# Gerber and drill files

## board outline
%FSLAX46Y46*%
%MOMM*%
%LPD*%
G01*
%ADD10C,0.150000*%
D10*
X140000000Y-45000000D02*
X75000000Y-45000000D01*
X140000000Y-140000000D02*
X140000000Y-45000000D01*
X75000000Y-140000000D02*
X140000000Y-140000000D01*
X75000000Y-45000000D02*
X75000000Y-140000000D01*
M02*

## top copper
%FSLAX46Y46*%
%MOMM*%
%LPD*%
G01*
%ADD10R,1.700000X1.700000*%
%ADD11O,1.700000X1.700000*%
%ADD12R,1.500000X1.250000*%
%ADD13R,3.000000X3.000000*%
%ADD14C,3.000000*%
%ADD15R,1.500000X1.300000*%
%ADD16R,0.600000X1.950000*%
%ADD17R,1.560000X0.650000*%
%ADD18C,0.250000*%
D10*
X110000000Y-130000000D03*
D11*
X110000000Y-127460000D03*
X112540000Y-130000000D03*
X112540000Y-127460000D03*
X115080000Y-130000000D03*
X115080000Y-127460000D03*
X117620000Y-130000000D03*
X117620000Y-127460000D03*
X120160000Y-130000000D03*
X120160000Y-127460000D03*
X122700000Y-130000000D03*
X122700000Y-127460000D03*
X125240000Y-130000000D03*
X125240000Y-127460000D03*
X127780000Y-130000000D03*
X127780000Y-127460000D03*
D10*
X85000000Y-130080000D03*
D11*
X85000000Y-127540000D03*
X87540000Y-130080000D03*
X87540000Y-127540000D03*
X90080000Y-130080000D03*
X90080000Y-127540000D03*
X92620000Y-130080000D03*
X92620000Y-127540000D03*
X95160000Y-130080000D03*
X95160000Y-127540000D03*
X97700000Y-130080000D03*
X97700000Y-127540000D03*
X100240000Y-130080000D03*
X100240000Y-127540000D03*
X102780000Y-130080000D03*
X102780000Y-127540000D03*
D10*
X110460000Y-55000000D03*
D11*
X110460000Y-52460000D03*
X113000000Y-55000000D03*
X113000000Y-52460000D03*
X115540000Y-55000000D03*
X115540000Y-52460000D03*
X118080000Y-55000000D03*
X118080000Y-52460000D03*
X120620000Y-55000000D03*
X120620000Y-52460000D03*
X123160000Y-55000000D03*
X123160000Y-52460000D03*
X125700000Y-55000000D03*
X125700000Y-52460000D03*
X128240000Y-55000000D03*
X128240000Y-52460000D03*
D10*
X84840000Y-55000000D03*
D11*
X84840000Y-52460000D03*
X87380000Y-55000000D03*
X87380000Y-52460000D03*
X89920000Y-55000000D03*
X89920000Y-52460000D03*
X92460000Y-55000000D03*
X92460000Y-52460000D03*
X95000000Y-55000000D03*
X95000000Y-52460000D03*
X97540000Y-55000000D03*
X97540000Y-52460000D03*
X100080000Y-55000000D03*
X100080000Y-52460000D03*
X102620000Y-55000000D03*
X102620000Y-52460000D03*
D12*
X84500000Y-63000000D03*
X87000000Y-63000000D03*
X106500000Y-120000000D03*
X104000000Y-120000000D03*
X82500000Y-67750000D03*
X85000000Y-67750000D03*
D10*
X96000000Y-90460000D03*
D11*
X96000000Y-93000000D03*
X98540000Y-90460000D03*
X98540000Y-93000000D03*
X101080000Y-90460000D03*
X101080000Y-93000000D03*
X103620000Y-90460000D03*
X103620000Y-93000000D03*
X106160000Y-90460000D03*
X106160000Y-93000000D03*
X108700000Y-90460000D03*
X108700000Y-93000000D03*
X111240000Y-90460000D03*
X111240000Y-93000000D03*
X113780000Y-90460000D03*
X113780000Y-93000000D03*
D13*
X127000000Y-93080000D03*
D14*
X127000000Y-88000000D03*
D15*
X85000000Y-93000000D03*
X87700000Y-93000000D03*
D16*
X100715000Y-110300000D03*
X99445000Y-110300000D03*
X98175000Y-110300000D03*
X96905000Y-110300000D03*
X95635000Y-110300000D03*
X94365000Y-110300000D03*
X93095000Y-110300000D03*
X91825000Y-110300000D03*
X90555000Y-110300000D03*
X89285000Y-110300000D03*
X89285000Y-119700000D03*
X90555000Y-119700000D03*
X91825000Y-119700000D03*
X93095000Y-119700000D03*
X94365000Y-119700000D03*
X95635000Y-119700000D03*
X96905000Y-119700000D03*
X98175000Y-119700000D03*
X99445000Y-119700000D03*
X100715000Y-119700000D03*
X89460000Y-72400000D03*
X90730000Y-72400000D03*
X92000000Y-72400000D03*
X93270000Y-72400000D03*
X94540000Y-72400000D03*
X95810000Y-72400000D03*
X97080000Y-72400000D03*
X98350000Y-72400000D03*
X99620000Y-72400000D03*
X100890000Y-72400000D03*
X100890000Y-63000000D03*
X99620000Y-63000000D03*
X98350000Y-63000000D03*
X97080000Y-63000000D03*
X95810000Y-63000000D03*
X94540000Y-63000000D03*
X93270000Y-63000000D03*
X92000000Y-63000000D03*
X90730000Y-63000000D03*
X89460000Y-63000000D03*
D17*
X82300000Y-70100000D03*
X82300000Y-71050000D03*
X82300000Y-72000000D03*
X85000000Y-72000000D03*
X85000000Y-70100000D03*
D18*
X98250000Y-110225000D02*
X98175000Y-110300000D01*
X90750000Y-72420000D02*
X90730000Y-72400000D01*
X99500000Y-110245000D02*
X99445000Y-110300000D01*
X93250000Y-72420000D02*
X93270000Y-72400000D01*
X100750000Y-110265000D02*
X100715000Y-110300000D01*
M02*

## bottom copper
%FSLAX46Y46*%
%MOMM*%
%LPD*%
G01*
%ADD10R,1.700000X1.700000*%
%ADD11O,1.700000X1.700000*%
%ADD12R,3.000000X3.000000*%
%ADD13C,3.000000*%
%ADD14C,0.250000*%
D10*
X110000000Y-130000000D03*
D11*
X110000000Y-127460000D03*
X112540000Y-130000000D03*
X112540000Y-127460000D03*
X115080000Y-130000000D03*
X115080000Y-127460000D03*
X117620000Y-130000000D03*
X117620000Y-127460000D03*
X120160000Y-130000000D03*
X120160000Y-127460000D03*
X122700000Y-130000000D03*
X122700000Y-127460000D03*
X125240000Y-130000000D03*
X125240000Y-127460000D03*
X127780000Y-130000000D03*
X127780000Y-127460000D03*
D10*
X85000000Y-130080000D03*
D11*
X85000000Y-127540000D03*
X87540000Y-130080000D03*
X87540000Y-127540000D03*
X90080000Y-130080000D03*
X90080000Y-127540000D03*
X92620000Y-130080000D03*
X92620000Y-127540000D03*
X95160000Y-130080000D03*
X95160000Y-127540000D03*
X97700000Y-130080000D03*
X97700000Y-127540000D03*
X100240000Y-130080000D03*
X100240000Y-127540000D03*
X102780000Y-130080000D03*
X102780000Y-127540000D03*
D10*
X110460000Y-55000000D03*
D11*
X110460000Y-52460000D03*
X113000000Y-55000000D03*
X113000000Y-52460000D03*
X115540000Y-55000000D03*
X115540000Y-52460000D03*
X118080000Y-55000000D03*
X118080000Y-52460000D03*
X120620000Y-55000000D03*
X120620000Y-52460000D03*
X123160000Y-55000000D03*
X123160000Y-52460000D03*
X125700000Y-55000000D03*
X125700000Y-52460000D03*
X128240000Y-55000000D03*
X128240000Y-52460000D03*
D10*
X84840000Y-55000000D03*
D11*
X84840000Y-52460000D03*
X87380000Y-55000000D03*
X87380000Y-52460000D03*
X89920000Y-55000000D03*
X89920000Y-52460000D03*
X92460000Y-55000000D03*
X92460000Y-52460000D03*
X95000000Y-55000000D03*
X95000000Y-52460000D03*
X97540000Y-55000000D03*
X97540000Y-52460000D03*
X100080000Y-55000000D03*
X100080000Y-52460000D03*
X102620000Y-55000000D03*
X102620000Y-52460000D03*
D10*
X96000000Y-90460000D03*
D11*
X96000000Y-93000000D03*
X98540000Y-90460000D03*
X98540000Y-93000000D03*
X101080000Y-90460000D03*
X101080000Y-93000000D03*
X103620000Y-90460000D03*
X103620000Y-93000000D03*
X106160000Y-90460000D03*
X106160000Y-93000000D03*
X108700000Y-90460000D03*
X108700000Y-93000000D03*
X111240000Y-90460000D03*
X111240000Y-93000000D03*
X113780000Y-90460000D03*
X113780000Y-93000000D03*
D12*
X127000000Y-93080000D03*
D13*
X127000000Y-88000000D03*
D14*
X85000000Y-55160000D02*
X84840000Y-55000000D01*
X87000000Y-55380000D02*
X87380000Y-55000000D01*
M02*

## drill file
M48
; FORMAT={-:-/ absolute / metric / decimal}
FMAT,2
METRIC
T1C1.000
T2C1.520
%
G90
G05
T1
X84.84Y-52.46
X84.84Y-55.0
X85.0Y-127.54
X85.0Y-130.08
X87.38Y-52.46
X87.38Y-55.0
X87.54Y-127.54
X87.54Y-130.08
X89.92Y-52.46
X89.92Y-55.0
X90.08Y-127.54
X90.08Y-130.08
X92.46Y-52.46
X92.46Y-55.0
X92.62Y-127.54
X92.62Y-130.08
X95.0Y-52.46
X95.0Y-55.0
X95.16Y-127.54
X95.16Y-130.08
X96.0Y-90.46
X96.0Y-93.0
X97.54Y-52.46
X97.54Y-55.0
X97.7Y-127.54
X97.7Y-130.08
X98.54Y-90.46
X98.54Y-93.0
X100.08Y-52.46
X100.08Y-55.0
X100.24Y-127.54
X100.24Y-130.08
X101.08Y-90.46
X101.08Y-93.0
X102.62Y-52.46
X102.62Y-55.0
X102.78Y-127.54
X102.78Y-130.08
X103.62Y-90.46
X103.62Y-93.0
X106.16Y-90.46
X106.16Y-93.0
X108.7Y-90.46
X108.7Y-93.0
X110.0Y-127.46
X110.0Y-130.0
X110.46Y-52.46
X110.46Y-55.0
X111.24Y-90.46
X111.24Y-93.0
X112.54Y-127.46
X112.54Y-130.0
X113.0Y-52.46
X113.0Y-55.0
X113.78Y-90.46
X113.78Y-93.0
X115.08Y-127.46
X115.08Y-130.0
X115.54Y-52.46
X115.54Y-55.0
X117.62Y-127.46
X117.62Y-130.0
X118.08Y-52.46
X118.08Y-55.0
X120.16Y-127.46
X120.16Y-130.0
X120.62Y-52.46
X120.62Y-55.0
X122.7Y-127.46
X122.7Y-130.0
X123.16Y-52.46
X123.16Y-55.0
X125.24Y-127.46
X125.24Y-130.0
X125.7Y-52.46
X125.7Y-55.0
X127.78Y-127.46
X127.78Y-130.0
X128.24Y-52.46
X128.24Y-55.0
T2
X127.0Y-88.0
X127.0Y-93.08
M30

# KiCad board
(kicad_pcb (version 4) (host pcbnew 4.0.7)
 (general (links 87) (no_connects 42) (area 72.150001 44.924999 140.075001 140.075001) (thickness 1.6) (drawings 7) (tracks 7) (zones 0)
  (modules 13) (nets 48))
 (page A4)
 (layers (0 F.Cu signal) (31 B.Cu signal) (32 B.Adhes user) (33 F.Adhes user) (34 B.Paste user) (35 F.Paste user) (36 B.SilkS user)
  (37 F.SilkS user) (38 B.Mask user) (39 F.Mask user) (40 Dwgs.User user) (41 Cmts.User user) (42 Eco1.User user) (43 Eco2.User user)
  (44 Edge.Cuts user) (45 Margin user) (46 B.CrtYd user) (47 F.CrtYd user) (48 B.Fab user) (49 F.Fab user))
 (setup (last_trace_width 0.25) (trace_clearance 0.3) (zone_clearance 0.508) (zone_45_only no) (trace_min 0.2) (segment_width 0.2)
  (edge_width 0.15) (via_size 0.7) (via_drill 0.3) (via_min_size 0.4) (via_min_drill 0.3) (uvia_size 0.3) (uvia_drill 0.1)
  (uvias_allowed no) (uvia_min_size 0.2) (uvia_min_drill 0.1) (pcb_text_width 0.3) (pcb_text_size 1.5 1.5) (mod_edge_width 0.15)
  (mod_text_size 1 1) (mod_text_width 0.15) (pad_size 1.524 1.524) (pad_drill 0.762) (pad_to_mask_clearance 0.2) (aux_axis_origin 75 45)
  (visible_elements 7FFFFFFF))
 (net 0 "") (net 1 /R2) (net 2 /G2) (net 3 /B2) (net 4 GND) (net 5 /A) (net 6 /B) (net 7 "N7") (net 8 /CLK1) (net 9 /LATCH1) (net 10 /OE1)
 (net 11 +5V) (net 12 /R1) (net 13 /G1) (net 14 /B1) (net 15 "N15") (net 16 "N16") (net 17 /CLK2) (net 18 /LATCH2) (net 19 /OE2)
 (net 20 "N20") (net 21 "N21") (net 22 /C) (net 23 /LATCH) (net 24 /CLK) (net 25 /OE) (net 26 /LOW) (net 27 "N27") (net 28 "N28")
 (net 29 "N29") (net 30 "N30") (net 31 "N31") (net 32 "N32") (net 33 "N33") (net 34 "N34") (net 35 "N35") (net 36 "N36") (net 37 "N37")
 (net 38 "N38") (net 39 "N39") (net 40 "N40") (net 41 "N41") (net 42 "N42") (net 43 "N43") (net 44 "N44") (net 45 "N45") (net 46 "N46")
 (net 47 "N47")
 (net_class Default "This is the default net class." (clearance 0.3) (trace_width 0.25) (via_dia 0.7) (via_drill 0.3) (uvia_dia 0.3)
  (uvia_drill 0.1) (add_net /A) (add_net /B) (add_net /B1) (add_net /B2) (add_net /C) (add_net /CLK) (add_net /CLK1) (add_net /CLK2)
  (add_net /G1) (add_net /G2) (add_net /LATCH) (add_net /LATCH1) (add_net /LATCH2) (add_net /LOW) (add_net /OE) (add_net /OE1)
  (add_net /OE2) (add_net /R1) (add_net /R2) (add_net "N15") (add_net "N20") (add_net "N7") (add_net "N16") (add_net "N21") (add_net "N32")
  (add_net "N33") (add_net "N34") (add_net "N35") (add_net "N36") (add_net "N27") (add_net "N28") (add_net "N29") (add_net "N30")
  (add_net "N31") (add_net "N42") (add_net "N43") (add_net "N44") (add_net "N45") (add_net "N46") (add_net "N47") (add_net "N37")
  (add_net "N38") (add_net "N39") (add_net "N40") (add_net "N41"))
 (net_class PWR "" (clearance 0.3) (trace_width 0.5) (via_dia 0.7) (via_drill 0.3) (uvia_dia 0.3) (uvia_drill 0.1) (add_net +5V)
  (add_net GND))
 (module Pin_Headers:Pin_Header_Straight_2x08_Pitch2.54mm (layer F.Cu) (at 110 130 90)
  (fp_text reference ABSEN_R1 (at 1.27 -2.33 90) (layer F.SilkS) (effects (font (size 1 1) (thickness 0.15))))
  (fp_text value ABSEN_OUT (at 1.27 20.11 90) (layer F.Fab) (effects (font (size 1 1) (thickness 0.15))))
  (pad 1 thru_hole rect (at 0 0 90) (size 1.7 1.7) (drill 1) (layers *.Cu *.Mask) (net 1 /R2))
  (pad 2 thru_hole oval (at 2.54 0 90) (size 1.7 1.7) (drill 1) (layers *.Cu *.Mask) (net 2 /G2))
  (pad 3 thru_hole oval (at 0 2.54 90) (size 1.7 1.7) (drill 1) (layers *.Cu *.Mask) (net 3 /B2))
  (pad 4 thru_hole oval (at 2.54 2.54 90) (size 1.7 1.7) (drill 1) (layers *.Cu *.Mask) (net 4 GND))
  (pad 5 thru_hole oval (at 0 5.08 90) (size 1.7 1.7) (drill 1) (layers *.Cu *.Mask) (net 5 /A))
  (pad 6 thru_hole oval (at 2.54 5.08 90) (size 1.7 1.7) (drill 1) (layers *.Cu *.Mask) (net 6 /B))
  (pad 7 thru_hole oval (at 0 7.62 90) (size 1.7 1.7) (drill 1) (layers *.Cu *.Mask) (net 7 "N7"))
  (pad 8 thru_hole oval (at 2.54 7.62 90) (size 1.7 1.7) (drill 1) (layers *.Cu *.Mask) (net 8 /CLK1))
  (pad 9 thru_hole oval (at 0 10.16 90) (size 1.7 1.7) (drill 1) (layers *.Cu *.Mask) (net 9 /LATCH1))
  (pad 10 thru_hole oval (at 2.54 10.16 90) (size 1.7 1.7) (drill 1) (layers *.Cu *.Mask) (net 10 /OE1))
  (pad 11 thru_hole oval (at 0 12.7 90) (size 1.7 1.7) (drill 1) (layers *.Cu *.Mask) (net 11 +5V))
  (pad 12 thru_hole oval (at 2.54 12.7 90) (size 1.7 1.7) (drill 1) (layers *.Cu *.Mask) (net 4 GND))
  (pad 13 thru_hole oval (at 0 15.24 90) (size 1.7 1.7) (drill 1) (layers *.Cu *.Mask) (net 11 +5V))
  (pad 14 thru_hole oval (at 2.54 15.24 90) (size 1.7 1.7) (drill 1) (layers *.Cu *.Mask) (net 4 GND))
  (pad 15 thru_hole oval (at 0 17.78 90) (size 1.7 1.7) (drill 1) (layers *.Cu *.Mask) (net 11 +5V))
  (pad 16 thru_hole oval (at 2.54 17.78 90) (size 1.7 1.7) (drill 1) (layers *.Cu *.Mask) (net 4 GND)))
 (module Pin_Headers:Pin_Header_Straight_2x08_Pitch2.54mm (layer F.Cu) (at 85 130.08 90)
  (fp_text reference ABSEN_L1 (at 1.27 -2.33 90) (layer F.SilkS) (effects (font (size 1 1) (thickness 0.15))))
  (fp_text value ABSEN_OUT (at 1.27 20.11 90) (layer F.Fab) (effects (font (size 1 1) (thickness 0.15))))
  (pad 1 thru_hole rect (at 0 0 90) (size 1.7 1.7) (drill 1) (layers *.Cu *.Mask) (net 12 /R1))
  (pad 2 thru_hole oval (at 2.54 0 90) (size 1.7 1.7) (drill 1) (layers *.Cu *.Mask) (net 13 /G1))
  (pad 3 thru_hole oval (at 0 2.54 90) (size 1.7 1.7) (drill 1) (layers *.Cu *.Mask) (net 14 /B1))
  (pad 4 thru_hole oval (at 2.54 2.54 90) (size 1.7 1.7) (drill 1) (layers *.Cu *.Mask) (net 4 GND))
  (pad 5 thru_hole oval (at 0 5.08 90) (size 1.7 1.7) (drill 1) (layers *.Cu *.Mask) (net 5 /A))
  (pad 6 thru_hole oval (at 2.54 5.08 90) (size 1.7 1.7) (drill 1) (layers *.Cu *.Mask) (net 6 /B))
  (pad 7 thru_hole oval (at 0 7.62 90) (size 1.7 1.7) (drill 1) (layers *.Cu *.Mask) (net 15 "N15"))
  (pad 8 thru_hole oval (at 2.54 7.62 90) (size 1.7 1.7) (drill 1) (layers *.Cu *.Mask) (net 8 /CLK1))
  (pad 9 thru_hole oval (at 0 10.16 90) (size 1.7 1.7) (drill 1) (layers *.Cu *.Mask) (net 9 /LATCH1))
  (pad 10 thru_hole oval (at 2.54 10.16 90) (size 1.7 1.7) (drill 1) (layers *.Cu *.Mask) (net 10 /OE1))
  (pad 11 thru_hole oval (at 0 12.7 90) (size 1.7 1.7) (drill 1) (layers *.Cu *.Mask) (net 11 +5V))
  (pad 12 thru_hole oval (at 2.54 12.7 90) (size 1.7 1.7) (drill 1) (layers *.Cu *.Mask) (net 4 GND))
  (pad 13 thru_hole oval (at 0 15.24 90) (size 1.7 1.7) (drill 1) (layers *.Cu *.Mask) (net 11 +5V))
  (pad 14 thru_hole oval (at 2.54 15.24 90) (size 1.7 1.7) (drill 1) (layers *.Cu *.Mask) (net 4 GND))
  (pad 15 thru_hole oval (at 0 17.78 90) (size 1.7 1.7) (drill 1) (layers *.Cu *.Mask) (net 11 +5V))
  (pad 16 thru_hole oval (at 2.54 17.78 90) (size 1.7 1.7) (drill 1) (layers *.Cu *.Mask) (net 4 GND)))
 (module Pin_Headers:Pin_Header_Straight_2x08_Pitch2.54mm (layer F.Cu) (at 110.46 55 90)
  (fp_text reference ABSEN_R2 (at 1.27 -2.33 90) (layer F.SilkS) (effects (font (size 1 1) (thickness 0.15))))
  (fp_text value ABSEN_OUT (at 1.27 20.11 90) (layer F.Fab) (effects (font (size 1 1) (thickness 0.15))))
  (pad 1 thru_hole rect (at 0 0 90) (size 1.7 1.7) (drill 1) (layers *.Cu *.Mask) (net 1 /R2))
  (pad 2 thru_hole oval (at 2.54 0 90) (size 1.7 1.7) (drill 1) (layers *.Cu *.Mask) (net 2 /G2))
  (pad 3 thru_hole oval (at 0 2.54 90) (size 1.7 1.7) (drill 1) (layers *.Cu *.Mask) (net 3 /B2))
  (pad 4 thru_hole oval (at 2.54 2.54 90) (size 1.7 1.7) (drill 1) (layers *.Cu *.Mask) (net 4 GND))
  (pad 5 thru_hole oval (at 0 5.08 90) (size 1.7 1.7) (drill 1) (layers *.Cu *.Mask) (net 5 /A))
  (pad 6 thru_hole oval (at 2.54 5.08 90) (size 1.7 1.7) (drill 1) (layers *.Cu *.Mask) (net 6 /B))
  (pad 7 thru_hole oval (at 0 7.62 90) (size 1.7 1.7) (drill 1) (layers *.Cu *.Mask) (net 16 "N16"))
  (pad 8 thru_hole oval (at 2.54 7.62 90) (size 1.7 1.7) (drill 1) (layers *.Cu *.Mask) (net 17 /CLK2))
  (pad 9 thru_hole oval (at 0 10.16 90) (size 1.7 1.7) (drill 1) (layers *.Cu *.Mask) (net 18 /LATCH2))
  (pad 10 thru_hole oval (at 2.54 10.16 90) (size 1.7 1.7) (drill 1) (layers *.Cu *.Mask) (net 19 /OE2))
  (pad 11 thru_hole oval (at 0 12.7 90) (size 1.7 1.7) (drill 1) (layers *.Cu *.Mask) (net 11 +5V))
  (pad 12 thru_hole oval (at 2.54 12.7 90) (size 1.7 1.7) (drill 1) (layers *.Cu *.Mask) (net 4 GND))
  (pad 13 thru_hole oval (at 0 15.24 90) (size 1.7 1.7) (drill 1) (layers *.Cu *.Mask) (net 11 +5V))
  (pad 14 thru_hole oval (at 2.54 15.24 90) (size 1.7 1.7) (drill 1) (layers *.Cu *.Mask) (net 4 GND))
  (pad 15 thru_hole oval (at 0 17.78 90) (size 1.7 1.7) (drill 1) (layers *.Cu *.Mask) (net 11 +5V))
  (pad 16 thru_hole oval (at 2.54 17.78 90) (size 1.7 1.7) (drill 1) (layers *.Cu *.Mask) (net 4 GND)))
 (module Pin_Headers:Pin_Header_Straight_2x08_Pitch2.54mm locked (layer F.Cu) (at 84.84 55 90)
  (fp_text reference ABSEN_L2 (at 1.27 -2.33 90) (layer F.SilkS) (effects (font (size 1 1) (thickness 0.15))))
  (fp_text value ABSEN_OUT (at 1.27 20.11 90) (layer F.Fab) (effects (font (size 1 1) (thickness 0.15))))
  (pad 1 thru_hole rect (at 0 0 90) (size 1.7 1.7) (drill 1) (layers *.Cu *.Mask) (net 12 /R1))
  (pad 2 thru_hole oval (at 2.54 0 90) (size 1.7 1.7) (drill 1) (layers *.Cu *.Mask) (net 13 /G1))
  (pad 3 thru_hole oval (at 0 2.54 90) (size 1.7 1.7) (drill 1) (layers *.Cu *.Mask) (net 14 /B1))
  (pad 4 thru_hole oval (at 2.54 2.54 90) (size 1.7 1.7) (drill 1) (layers *.Cu *.Mask) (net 4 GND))
  (pad 5 thru_hole oval (at 0 5.08 90) (size 1.7 1.7) (drill 1) (layers *.Cu *.Mask) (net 5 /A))
  (pad 6 thru_hole oval (at 2.54 5.08 90) (size 1.7 1.7) (drill 1) (layers *.Cu *.Mask) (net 6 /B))
  (pad 7 thru_hole oval (at 0 7.62 90) (size 1.7 1.7) (drill 1) (layers *.Cu *.Mask) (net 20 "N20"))
  (pad 8 thru_hole oval (at 2.54 7.62 90) (size 1.7 1.7) (drill 1) (layers *.Cu *.Mask) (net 17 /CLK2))
  (pad 9 thru_hole oval (at 0 10.16 90) (size 1.7 1.7) (drill 1) (layers *.Cu *.Mask) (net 18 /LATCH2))
  (pad 10 thru_hole oval (at 2.54 10.16 90) (size 1.7 1.7) (drill 1) (layers *.Cu *.Mask) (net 19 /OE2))
  (pad 11 thru_hole oval (at 0 12.7 90) (size 1.7 1.7) (drill 1) (layers *.Cu *.Mask) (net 11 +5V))
  (pad 12 thru_hole oval (at 2.54 12.7 90) (size 1.7 1.7) (drill 1) (layers *.Cu *.Mask) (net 4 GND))
  (pad 13 thru_hole oval (at 0 15.24 90) (size 1.7 1.7) (drill 1) (layers *.Cu *.Mask) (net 11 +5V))
  (pad 14 thru_hole oval (at 2.54 15.24 90) (size 1.7 1.7) (drill 1) (layers *.Cu *.Mask) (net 4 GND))
  (pad 15 thru_hole oval (at 0 17.78 90) (size 1.7 1.7) (drill 1) (layers *.Cu *.Mask) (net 11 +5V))
  (pad 16 thru_hole oval (at 2.54 17.78 90) (size 1.7 1.7) (drill 1) (layers *.Cu *.Mask) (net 4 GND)))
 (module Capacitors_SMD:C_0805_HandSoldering (layer F.Cu) (at 85.75 63)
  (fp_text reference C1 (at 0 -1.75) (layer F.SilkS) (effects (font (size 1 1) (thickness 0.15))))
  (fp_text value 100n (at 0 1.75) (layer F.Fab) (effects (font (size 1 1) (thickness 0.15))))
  (pad 1 smd rect (at -1.25 0) (size 1.5 1.25) (layers F.Cu F.Paste F.Mask) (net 4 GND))
  (pad 2 smd rect (at 1.25 0) (size 1.5 1.25) (layers F.Cu F.Paste F.Mask) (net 11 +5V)))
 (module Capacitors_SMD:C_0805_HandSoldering (layer F.Cu) (at 105.25 120 180)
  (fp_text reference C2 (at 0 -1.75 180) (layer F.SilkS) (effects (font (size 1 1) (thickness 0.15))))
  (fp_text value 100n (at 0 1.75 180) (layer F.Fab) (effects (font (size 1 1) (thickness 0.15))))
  (pad 1 smd rect (at -1.25 0 180) (size 1.5 1.25) (layers F.Cu F.Paste F.Mask) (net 4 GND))
  (pad 2 smd rect (at 1.25 0 180) (size 1.5 1.25) (layers F.Cu F.Paste F.Mask) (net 11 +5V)))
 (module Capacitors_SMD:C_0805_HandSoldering (layer F.Cu) (at 83.75 67.75)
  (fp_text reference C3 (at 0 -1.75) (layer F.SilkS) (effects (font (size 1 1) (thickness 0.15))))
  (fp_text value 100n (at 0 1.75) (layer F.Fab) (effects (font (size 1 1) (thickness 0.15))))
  (pad 1 smd rect (at -1.25 0) (size 1.5 1.25) (layers F.Cu F.Paste F.Mask) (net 4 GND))
  (pad 2 smd rect (at 1.25 0) (size 1.5 1.25) (layers F.Cu F.Paste F.Mask) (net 11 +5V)))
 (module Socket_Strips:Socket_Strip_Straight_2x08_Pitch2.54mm (layer F.Cu) (at 96 90.46 90)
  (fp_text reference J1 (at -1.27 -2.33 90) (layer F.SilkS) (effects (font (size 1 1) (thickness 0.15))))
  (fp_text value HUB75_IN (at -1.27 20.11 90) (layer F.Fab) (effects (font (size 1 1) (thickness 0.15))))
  (pad 1 thru_hole rect (at 0 0 90) (size 1.7 1.7) (drill 1) (layers *.Cu *.Mask) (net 13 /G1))
  (pad 2 thru_hole oval (at -2.54 0 90) (size 1.7 1.7) (drill 1) (layers *.Cu *.Mask) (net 12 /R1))
  (pad 3 thru_hole oval (at 0 2.54 90) (size 1.7 1.7) (drill 1) (layers *.Cu *.Mask) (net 4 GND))
  (pad 4 thru_hole oval (at -2.54 2.54 90) (size 1.7 1.7) (drill 1) (layers *.Cu *.Mask) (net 14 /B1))
  (pad 5 thru_hole oval (at 0 5.08 90) (size 1.7 1.7) (drill 1) (layers *.Cu *.Mask) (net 2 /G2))
  (pad 6 thru_hole oval (at -2.54 5.08 90) (size 1.7 1.7) (drill 1) (layers *.Cu *.Mask) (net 1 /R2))
  (pad 7 thru_hole oval (at 0 7.62 90) (size 1.7 1.7) (drill 1) (layers *.Cu *.Mask) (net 4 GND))
  (pad 8 thru_hole oval (at -2.54 7.62 90) (size 1.7 1.7) (drill 1) (layers *.Cu *.Mask) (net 3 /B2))
  (pad 9 thru_hole oval (at 0 10.16 90) (size 1.7 1.7) (drill 1) (layers *.Cu *.Mask) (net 6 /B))
  (pad 10 thru_hole oval (at -2.54 10.16 90) (size 1.7 1.7) (drill 1) (layers *.Cu *.Mask) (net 5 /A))
  (pad 11 thru_hole oval (at 0 12.7 90) (size 1.7 1.7) (drill 1) (layers *.Cu *.Mask) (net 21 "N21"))
  (pad 12 thru_hole oval (at -2.54 12.7 90) (size 1.7 1.7) (drill 1) (layers *.Cu *.Mask) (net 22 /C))
  (pad 13 thru_hole oval (at 0 15.24 90) (size 1.7 1.7) (drill 1) (layers *.Cu *.Mask) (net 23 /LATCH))
  (pad 14 thru_hole oval (at -2.54 15.24 90) (size 1.7 1.7) (drill 1) (layers *.Cu *.Mask) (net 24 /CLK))
  (pad 15 thru_hole oval (at 0 17.78 90) (size 1.7 1.7) (drill 1) (layers *.Cu *.Mask) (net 4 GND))
  (pad 16 thru_hole oval (at -2.54 17.78 90) (size 1.7 1.7) (drill 1) (layers *.Cu *.Mask) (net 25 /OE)))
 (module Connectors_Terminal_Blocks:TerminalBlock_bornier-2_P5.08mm (layer F.Cu) (at 127 93.08 90)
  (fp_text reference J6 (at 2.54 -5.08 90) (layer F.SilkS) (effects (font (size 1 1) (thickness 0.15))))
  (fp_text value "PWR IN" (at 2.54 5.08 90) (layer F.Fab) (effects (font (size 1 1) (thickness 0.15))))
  (pad 1 thru_hole rect (at 0 0 90) (size 3 3) (drill 1.52) (layers *.Cu *.Mask) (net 11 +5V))
  (pad 2 thru_hole circle (at 5.08 0 90) (size 3 3) (drill 1.52) (layers *.Cu *.Mask) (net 4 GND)))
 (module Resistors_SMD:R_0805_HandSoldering (layer F.Cu) (at 86.35 93)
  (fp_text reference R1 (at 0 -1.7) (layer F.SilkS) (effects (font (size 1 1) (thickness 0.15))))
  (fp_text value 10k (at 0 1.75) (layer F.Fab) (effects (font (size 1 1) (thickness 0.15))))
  (pad 1 smd rect (at -1.35 0) (size 1.5 1.3) (layers F.Cu F.Paste F.Mask) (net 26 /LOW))
  (pad 2 smd rect (at 1.35 0) (size 1.5 1.3) (layers F.Cu F.Paste F.Mask) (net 4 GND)))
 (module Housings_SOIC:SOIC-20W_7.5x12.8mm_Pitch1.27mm (layer F.Cu) (at 95 115 270)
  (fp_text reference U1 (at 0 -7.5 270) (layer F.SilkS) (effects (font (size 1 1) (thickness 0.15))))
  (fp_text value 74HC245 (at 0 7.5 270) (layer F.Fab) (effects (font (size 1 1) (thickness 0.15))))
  (pad 1 smd rect (at -4.7 -5.715 270) (size 1.95 0.6) (layers F.Cu F.Paste F.Mask) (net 26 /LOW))
  (pad 2 smd rect (at -4.7 -4.445 270) (size 1.95 0.6) (layers F.Cu F.Paste F.Mask) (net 24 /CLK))
  (pad 3 smd rect (at -4.7 -3.175 270) (size 1.95 0.6) (layers F.Cu F.Paste F.Mask) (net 23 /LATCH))
  (pad 4 smd rect (at -4.7 -1.905 270) (size 1.95 0.6) (layers F.Cu F.Paste F.Mask) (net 25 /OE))
  (pad 5 smd rect (at -4.7 -0.635 270) (size 1.95 0.6) (layers F.Cu F.Paste F.Mask) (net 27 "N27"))
  (pad 6 smd rect (at -4.7 0.635 270) (size 1.95 0.6) (layers F.Cu F.Paste F.Mask) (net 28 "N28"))
  (pad 7 smd rect (at -4.7 1.905 270) (size 1.95 0.6) (layers F.Cu F.Paste F.Mask) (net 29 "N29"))
  (pad 8 smd rect (at -4.7 3.175 270) (size 1.95 0.6) (layers F.Cu F.Paste F.Mask) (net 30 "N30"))
  (pad 9 smd rect (at -4.7 4.445 270) (size 1.95 0.6) (layers F.Cu F.Paste F.Mask) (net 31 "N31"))
  (pad 10 smd rect (at -4.7 5.715 270) (size 1.95 0.6) (layers F.Cu F.Paste F.Mask) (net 4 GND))
  (pad 11 smd rect (at 4.7 5.715 270) (size 1.95 0.6) (layers F.Cu F.Paste F.Mask) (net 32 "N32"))
  (pad 12 smd rect (at 4.7 4.445 270) (size 1.95 0.6) (layers F.Cu F.Paste F.Mask) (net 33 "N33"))
  (pad 13 smd rect (at 4.7 3.175 270) (size 1.95 0.6) (layers F.Cu F.Paste F.Mask) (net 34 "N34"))
  (pad 14 smd rect (at 4.7 1.905 270) (size 1.95 0.6) (layers F.Cu F.Paste F.Mask) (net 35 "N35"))
  (pad 15 smd rect (at 4.7 0.635 270) (size 1.95 0.6) (layers F.Cu F.Paste F.Mask) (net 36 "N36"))
  (pad 16 smd rect (at 4.7 -0.635 270) (size 1.95 0.6) (layers F.Cu F.Paste F.Mask) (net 10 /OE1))
  (pad 17 smd rect (at 4.7 -1.905 270) (size 1.95 0.6) (layers F.Cu F.Paste F.Mask) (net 9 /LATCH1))
  (pad 18 smd rect (at 4.7 -3.175 270) (size 1.95 0.6) (layers F.Cu F.Paste F.Mask) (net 8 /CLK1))
  (pad 19 smd rect (at 4.7 -4.445 270) (size 1.95 0.6) (layers F.Cu F.Paste F.Mask) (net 22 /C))
  (pad 20 smd rect (at 4.7 -5.715 270) (size 1.95 0.6) (layers F.Cu F.Paste F.Mask) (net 11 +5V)))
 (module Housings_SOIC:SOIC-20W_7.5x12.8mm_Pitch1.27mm (layer F.Cu) (at 95.175 67.7 90)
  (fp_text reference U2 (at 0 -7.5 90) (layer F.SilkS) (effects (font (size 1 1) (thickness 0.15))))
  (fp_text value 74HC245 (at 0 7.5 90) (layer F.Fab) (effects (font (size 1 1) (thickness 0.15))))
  (pad 1 smd rect (at -4.7 -5.715 90) (size 1.95 0.6) (layers F.Cu F.Paste F.Mask) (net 26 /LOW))
  (pad 2 smd rect (at -4.7 -4.445 90) (size 1.95 0.6) (layers F.Cu F.Paste F.Mask) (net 24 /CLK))
  (pad 3 smd rect (at -4.7 -3.175 90) (size 1.95 0.6) (layers F.Cu F.Paste F.Mask) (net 23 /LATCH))
  (pad 4 smd rect (at -4.7 -1.905 90) (size 1.95 0.6) (layers F.Cu F.Paste F.Mask) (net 25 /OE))
  (pad 5 smd rect (at -4.7 -0.635 90) (size 1.95 0.6) (layers F.Cu F.Paste F.Mask) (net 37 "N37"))
  (pad 6 smd rect (at -4.7 0.635 90) (size 1.95 0.6) (layers F.Cu F.Paste F.Mask) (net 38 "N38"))
  (pad 7 smd rect (at -4.7 1.905 90) (size 1.95 0.6) (layers F.Cu F.Paste F.Mask) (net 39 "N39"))
  (pad 8 smd rect (at -4.7 3.175 90) (size 1.95 0.6) (layers F.Cu F.Paste F.Mask) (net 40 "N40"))
  (pad 9 smd rect (at -4.7 4.445 90) (size 1.95 0.6) (layers F.Cu F.Paste F.Mask) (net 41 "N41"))
  (pad 10 smd rect (at -4.7 5.715 90) (size 1.95 0.6) (layers F.Cu F.Paste F.Mask) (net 4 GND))
  (pad 11 smd rect (at 4.7 5.715 90) (size 1.95 0.6) (layers F.Cu F.Paste F.Mask) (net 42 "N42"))
  (pad 12 smd rect (at 4.7 4.445 90) (size 1.95 0.6) (layers F.Cu F.Paste F.Mask) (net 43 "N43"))
  (pad 13 smd rect (at 4.7 3.175 90) (size 1.95 0.6) (layers F.Cu F.Paste F.Mask) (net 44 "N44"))
  (pad 14 smd rect (at 4.7 1.905 90) (size 1.95 0.6) (layers F.Cu F.Paste F.Mask) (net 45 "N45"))
  (pad 15 smd rect (at 4.7 0.635 90) (size 1.95 0.6) (layers F.Cu F.Paste F.Mask) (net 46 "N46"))
  (pad 16 smd rect (at 4.7 -0.635 90) (size 1.95 0.6) (layers F.Cu F.Paste F.Mask) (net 19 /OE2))
  (pad 17 smd rect (at 4.7 -1.905 90) (size 1.95 0.6) (layers F.Cu F.Paste F.Mask) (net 18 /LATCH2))
  (pad 18 smd rect (at 4.7 -3.175 90) (size 1.95 0.6) (layers F.Cu F.Paste F.Mask) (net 17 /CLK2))
  (pad 19 smd rect (at 4.7 -4.445 90) (size 1.95 0.6) (layers F.Cu F.Paste F.Mask) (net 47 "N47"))
  (pad 20 smd rect (at 4.7 -5.715 90) (size 1.95 0.6) (layers F.Cu F.Paste F.Mask) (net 11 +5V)))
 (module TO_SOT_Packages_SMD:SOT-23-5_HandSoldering (layer F.Cu) (at 83.65 71.05)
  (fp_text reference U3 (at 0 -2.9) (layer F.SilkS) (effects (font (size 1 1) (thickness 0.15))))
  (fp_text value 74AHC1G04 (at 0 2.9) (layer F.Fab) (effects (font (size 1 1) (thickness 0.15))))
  (pad 1 smd rect (at -1.35 -0.95) (size 1.56 0.65) (layers F.Cu F.Paste F.Mask))
  (pad 2 smd rect (at -1.35 0) (size 1.56 0.65) (layers F.Cu F.Paste F.Mask) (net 22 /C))
  (pad 3 smd rect (at -1.35 0.95) (size 1.56 0.65) (layers F.Cu F.Paste F.Mask) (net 4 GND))
  (pad 4 smd rect (at 1.35 0.95) (size 1.56 0.65) (layers F.Cu F.Paste F.Mask) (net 47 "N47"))
  (pad 5 smd rect (at 1.35 -0.95) (size 1.56 0.65) (layers F.Cu F.Paste F.Mask) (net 11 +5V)))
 (gr_line (start 140 45) (end 75 45) (layer Edge.Cuts) (width 0.15))
 (gr_line (start 140 140) (end 140 45) (layer Edge.Cuts) (width 0.15))
 (gr_line (start 75 140) (end 140 140) (layer Edge.Cuts) (width 0.15))
 (gr_line (start 75 45) (end 75 140) (layer Edge.Cuts) (width 0.15))
 (segment (start 85 55.16) (end 84.84 55) (width 0.25) (layer B.Cu) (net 12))
 (segment (start 87 55.38) (end 87.38 55) (width 0.25) (layer B.Cu) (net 14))
 (segment (start 98.25 110.225) (end 98.175 110.3) (width 0.25) (layer F.Cu) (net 23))
 (segment (start 90.75 72.42) (end 90.73 72.4) (width 0.25) (layer F.Cu) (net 24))
 (segment (start 99.5 110.245) (end 99.445 110.3) (width 0.25) (layer F.Cu) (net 24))
 (segment (start 93.25 72.42) (end 93.27 72.4) (width 0.25) (layer F.Cu) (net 25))
 (segment (start 100.75 110.265) (end 100.715 110.3) (width 0.25) (layer F.Cu) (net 26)))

